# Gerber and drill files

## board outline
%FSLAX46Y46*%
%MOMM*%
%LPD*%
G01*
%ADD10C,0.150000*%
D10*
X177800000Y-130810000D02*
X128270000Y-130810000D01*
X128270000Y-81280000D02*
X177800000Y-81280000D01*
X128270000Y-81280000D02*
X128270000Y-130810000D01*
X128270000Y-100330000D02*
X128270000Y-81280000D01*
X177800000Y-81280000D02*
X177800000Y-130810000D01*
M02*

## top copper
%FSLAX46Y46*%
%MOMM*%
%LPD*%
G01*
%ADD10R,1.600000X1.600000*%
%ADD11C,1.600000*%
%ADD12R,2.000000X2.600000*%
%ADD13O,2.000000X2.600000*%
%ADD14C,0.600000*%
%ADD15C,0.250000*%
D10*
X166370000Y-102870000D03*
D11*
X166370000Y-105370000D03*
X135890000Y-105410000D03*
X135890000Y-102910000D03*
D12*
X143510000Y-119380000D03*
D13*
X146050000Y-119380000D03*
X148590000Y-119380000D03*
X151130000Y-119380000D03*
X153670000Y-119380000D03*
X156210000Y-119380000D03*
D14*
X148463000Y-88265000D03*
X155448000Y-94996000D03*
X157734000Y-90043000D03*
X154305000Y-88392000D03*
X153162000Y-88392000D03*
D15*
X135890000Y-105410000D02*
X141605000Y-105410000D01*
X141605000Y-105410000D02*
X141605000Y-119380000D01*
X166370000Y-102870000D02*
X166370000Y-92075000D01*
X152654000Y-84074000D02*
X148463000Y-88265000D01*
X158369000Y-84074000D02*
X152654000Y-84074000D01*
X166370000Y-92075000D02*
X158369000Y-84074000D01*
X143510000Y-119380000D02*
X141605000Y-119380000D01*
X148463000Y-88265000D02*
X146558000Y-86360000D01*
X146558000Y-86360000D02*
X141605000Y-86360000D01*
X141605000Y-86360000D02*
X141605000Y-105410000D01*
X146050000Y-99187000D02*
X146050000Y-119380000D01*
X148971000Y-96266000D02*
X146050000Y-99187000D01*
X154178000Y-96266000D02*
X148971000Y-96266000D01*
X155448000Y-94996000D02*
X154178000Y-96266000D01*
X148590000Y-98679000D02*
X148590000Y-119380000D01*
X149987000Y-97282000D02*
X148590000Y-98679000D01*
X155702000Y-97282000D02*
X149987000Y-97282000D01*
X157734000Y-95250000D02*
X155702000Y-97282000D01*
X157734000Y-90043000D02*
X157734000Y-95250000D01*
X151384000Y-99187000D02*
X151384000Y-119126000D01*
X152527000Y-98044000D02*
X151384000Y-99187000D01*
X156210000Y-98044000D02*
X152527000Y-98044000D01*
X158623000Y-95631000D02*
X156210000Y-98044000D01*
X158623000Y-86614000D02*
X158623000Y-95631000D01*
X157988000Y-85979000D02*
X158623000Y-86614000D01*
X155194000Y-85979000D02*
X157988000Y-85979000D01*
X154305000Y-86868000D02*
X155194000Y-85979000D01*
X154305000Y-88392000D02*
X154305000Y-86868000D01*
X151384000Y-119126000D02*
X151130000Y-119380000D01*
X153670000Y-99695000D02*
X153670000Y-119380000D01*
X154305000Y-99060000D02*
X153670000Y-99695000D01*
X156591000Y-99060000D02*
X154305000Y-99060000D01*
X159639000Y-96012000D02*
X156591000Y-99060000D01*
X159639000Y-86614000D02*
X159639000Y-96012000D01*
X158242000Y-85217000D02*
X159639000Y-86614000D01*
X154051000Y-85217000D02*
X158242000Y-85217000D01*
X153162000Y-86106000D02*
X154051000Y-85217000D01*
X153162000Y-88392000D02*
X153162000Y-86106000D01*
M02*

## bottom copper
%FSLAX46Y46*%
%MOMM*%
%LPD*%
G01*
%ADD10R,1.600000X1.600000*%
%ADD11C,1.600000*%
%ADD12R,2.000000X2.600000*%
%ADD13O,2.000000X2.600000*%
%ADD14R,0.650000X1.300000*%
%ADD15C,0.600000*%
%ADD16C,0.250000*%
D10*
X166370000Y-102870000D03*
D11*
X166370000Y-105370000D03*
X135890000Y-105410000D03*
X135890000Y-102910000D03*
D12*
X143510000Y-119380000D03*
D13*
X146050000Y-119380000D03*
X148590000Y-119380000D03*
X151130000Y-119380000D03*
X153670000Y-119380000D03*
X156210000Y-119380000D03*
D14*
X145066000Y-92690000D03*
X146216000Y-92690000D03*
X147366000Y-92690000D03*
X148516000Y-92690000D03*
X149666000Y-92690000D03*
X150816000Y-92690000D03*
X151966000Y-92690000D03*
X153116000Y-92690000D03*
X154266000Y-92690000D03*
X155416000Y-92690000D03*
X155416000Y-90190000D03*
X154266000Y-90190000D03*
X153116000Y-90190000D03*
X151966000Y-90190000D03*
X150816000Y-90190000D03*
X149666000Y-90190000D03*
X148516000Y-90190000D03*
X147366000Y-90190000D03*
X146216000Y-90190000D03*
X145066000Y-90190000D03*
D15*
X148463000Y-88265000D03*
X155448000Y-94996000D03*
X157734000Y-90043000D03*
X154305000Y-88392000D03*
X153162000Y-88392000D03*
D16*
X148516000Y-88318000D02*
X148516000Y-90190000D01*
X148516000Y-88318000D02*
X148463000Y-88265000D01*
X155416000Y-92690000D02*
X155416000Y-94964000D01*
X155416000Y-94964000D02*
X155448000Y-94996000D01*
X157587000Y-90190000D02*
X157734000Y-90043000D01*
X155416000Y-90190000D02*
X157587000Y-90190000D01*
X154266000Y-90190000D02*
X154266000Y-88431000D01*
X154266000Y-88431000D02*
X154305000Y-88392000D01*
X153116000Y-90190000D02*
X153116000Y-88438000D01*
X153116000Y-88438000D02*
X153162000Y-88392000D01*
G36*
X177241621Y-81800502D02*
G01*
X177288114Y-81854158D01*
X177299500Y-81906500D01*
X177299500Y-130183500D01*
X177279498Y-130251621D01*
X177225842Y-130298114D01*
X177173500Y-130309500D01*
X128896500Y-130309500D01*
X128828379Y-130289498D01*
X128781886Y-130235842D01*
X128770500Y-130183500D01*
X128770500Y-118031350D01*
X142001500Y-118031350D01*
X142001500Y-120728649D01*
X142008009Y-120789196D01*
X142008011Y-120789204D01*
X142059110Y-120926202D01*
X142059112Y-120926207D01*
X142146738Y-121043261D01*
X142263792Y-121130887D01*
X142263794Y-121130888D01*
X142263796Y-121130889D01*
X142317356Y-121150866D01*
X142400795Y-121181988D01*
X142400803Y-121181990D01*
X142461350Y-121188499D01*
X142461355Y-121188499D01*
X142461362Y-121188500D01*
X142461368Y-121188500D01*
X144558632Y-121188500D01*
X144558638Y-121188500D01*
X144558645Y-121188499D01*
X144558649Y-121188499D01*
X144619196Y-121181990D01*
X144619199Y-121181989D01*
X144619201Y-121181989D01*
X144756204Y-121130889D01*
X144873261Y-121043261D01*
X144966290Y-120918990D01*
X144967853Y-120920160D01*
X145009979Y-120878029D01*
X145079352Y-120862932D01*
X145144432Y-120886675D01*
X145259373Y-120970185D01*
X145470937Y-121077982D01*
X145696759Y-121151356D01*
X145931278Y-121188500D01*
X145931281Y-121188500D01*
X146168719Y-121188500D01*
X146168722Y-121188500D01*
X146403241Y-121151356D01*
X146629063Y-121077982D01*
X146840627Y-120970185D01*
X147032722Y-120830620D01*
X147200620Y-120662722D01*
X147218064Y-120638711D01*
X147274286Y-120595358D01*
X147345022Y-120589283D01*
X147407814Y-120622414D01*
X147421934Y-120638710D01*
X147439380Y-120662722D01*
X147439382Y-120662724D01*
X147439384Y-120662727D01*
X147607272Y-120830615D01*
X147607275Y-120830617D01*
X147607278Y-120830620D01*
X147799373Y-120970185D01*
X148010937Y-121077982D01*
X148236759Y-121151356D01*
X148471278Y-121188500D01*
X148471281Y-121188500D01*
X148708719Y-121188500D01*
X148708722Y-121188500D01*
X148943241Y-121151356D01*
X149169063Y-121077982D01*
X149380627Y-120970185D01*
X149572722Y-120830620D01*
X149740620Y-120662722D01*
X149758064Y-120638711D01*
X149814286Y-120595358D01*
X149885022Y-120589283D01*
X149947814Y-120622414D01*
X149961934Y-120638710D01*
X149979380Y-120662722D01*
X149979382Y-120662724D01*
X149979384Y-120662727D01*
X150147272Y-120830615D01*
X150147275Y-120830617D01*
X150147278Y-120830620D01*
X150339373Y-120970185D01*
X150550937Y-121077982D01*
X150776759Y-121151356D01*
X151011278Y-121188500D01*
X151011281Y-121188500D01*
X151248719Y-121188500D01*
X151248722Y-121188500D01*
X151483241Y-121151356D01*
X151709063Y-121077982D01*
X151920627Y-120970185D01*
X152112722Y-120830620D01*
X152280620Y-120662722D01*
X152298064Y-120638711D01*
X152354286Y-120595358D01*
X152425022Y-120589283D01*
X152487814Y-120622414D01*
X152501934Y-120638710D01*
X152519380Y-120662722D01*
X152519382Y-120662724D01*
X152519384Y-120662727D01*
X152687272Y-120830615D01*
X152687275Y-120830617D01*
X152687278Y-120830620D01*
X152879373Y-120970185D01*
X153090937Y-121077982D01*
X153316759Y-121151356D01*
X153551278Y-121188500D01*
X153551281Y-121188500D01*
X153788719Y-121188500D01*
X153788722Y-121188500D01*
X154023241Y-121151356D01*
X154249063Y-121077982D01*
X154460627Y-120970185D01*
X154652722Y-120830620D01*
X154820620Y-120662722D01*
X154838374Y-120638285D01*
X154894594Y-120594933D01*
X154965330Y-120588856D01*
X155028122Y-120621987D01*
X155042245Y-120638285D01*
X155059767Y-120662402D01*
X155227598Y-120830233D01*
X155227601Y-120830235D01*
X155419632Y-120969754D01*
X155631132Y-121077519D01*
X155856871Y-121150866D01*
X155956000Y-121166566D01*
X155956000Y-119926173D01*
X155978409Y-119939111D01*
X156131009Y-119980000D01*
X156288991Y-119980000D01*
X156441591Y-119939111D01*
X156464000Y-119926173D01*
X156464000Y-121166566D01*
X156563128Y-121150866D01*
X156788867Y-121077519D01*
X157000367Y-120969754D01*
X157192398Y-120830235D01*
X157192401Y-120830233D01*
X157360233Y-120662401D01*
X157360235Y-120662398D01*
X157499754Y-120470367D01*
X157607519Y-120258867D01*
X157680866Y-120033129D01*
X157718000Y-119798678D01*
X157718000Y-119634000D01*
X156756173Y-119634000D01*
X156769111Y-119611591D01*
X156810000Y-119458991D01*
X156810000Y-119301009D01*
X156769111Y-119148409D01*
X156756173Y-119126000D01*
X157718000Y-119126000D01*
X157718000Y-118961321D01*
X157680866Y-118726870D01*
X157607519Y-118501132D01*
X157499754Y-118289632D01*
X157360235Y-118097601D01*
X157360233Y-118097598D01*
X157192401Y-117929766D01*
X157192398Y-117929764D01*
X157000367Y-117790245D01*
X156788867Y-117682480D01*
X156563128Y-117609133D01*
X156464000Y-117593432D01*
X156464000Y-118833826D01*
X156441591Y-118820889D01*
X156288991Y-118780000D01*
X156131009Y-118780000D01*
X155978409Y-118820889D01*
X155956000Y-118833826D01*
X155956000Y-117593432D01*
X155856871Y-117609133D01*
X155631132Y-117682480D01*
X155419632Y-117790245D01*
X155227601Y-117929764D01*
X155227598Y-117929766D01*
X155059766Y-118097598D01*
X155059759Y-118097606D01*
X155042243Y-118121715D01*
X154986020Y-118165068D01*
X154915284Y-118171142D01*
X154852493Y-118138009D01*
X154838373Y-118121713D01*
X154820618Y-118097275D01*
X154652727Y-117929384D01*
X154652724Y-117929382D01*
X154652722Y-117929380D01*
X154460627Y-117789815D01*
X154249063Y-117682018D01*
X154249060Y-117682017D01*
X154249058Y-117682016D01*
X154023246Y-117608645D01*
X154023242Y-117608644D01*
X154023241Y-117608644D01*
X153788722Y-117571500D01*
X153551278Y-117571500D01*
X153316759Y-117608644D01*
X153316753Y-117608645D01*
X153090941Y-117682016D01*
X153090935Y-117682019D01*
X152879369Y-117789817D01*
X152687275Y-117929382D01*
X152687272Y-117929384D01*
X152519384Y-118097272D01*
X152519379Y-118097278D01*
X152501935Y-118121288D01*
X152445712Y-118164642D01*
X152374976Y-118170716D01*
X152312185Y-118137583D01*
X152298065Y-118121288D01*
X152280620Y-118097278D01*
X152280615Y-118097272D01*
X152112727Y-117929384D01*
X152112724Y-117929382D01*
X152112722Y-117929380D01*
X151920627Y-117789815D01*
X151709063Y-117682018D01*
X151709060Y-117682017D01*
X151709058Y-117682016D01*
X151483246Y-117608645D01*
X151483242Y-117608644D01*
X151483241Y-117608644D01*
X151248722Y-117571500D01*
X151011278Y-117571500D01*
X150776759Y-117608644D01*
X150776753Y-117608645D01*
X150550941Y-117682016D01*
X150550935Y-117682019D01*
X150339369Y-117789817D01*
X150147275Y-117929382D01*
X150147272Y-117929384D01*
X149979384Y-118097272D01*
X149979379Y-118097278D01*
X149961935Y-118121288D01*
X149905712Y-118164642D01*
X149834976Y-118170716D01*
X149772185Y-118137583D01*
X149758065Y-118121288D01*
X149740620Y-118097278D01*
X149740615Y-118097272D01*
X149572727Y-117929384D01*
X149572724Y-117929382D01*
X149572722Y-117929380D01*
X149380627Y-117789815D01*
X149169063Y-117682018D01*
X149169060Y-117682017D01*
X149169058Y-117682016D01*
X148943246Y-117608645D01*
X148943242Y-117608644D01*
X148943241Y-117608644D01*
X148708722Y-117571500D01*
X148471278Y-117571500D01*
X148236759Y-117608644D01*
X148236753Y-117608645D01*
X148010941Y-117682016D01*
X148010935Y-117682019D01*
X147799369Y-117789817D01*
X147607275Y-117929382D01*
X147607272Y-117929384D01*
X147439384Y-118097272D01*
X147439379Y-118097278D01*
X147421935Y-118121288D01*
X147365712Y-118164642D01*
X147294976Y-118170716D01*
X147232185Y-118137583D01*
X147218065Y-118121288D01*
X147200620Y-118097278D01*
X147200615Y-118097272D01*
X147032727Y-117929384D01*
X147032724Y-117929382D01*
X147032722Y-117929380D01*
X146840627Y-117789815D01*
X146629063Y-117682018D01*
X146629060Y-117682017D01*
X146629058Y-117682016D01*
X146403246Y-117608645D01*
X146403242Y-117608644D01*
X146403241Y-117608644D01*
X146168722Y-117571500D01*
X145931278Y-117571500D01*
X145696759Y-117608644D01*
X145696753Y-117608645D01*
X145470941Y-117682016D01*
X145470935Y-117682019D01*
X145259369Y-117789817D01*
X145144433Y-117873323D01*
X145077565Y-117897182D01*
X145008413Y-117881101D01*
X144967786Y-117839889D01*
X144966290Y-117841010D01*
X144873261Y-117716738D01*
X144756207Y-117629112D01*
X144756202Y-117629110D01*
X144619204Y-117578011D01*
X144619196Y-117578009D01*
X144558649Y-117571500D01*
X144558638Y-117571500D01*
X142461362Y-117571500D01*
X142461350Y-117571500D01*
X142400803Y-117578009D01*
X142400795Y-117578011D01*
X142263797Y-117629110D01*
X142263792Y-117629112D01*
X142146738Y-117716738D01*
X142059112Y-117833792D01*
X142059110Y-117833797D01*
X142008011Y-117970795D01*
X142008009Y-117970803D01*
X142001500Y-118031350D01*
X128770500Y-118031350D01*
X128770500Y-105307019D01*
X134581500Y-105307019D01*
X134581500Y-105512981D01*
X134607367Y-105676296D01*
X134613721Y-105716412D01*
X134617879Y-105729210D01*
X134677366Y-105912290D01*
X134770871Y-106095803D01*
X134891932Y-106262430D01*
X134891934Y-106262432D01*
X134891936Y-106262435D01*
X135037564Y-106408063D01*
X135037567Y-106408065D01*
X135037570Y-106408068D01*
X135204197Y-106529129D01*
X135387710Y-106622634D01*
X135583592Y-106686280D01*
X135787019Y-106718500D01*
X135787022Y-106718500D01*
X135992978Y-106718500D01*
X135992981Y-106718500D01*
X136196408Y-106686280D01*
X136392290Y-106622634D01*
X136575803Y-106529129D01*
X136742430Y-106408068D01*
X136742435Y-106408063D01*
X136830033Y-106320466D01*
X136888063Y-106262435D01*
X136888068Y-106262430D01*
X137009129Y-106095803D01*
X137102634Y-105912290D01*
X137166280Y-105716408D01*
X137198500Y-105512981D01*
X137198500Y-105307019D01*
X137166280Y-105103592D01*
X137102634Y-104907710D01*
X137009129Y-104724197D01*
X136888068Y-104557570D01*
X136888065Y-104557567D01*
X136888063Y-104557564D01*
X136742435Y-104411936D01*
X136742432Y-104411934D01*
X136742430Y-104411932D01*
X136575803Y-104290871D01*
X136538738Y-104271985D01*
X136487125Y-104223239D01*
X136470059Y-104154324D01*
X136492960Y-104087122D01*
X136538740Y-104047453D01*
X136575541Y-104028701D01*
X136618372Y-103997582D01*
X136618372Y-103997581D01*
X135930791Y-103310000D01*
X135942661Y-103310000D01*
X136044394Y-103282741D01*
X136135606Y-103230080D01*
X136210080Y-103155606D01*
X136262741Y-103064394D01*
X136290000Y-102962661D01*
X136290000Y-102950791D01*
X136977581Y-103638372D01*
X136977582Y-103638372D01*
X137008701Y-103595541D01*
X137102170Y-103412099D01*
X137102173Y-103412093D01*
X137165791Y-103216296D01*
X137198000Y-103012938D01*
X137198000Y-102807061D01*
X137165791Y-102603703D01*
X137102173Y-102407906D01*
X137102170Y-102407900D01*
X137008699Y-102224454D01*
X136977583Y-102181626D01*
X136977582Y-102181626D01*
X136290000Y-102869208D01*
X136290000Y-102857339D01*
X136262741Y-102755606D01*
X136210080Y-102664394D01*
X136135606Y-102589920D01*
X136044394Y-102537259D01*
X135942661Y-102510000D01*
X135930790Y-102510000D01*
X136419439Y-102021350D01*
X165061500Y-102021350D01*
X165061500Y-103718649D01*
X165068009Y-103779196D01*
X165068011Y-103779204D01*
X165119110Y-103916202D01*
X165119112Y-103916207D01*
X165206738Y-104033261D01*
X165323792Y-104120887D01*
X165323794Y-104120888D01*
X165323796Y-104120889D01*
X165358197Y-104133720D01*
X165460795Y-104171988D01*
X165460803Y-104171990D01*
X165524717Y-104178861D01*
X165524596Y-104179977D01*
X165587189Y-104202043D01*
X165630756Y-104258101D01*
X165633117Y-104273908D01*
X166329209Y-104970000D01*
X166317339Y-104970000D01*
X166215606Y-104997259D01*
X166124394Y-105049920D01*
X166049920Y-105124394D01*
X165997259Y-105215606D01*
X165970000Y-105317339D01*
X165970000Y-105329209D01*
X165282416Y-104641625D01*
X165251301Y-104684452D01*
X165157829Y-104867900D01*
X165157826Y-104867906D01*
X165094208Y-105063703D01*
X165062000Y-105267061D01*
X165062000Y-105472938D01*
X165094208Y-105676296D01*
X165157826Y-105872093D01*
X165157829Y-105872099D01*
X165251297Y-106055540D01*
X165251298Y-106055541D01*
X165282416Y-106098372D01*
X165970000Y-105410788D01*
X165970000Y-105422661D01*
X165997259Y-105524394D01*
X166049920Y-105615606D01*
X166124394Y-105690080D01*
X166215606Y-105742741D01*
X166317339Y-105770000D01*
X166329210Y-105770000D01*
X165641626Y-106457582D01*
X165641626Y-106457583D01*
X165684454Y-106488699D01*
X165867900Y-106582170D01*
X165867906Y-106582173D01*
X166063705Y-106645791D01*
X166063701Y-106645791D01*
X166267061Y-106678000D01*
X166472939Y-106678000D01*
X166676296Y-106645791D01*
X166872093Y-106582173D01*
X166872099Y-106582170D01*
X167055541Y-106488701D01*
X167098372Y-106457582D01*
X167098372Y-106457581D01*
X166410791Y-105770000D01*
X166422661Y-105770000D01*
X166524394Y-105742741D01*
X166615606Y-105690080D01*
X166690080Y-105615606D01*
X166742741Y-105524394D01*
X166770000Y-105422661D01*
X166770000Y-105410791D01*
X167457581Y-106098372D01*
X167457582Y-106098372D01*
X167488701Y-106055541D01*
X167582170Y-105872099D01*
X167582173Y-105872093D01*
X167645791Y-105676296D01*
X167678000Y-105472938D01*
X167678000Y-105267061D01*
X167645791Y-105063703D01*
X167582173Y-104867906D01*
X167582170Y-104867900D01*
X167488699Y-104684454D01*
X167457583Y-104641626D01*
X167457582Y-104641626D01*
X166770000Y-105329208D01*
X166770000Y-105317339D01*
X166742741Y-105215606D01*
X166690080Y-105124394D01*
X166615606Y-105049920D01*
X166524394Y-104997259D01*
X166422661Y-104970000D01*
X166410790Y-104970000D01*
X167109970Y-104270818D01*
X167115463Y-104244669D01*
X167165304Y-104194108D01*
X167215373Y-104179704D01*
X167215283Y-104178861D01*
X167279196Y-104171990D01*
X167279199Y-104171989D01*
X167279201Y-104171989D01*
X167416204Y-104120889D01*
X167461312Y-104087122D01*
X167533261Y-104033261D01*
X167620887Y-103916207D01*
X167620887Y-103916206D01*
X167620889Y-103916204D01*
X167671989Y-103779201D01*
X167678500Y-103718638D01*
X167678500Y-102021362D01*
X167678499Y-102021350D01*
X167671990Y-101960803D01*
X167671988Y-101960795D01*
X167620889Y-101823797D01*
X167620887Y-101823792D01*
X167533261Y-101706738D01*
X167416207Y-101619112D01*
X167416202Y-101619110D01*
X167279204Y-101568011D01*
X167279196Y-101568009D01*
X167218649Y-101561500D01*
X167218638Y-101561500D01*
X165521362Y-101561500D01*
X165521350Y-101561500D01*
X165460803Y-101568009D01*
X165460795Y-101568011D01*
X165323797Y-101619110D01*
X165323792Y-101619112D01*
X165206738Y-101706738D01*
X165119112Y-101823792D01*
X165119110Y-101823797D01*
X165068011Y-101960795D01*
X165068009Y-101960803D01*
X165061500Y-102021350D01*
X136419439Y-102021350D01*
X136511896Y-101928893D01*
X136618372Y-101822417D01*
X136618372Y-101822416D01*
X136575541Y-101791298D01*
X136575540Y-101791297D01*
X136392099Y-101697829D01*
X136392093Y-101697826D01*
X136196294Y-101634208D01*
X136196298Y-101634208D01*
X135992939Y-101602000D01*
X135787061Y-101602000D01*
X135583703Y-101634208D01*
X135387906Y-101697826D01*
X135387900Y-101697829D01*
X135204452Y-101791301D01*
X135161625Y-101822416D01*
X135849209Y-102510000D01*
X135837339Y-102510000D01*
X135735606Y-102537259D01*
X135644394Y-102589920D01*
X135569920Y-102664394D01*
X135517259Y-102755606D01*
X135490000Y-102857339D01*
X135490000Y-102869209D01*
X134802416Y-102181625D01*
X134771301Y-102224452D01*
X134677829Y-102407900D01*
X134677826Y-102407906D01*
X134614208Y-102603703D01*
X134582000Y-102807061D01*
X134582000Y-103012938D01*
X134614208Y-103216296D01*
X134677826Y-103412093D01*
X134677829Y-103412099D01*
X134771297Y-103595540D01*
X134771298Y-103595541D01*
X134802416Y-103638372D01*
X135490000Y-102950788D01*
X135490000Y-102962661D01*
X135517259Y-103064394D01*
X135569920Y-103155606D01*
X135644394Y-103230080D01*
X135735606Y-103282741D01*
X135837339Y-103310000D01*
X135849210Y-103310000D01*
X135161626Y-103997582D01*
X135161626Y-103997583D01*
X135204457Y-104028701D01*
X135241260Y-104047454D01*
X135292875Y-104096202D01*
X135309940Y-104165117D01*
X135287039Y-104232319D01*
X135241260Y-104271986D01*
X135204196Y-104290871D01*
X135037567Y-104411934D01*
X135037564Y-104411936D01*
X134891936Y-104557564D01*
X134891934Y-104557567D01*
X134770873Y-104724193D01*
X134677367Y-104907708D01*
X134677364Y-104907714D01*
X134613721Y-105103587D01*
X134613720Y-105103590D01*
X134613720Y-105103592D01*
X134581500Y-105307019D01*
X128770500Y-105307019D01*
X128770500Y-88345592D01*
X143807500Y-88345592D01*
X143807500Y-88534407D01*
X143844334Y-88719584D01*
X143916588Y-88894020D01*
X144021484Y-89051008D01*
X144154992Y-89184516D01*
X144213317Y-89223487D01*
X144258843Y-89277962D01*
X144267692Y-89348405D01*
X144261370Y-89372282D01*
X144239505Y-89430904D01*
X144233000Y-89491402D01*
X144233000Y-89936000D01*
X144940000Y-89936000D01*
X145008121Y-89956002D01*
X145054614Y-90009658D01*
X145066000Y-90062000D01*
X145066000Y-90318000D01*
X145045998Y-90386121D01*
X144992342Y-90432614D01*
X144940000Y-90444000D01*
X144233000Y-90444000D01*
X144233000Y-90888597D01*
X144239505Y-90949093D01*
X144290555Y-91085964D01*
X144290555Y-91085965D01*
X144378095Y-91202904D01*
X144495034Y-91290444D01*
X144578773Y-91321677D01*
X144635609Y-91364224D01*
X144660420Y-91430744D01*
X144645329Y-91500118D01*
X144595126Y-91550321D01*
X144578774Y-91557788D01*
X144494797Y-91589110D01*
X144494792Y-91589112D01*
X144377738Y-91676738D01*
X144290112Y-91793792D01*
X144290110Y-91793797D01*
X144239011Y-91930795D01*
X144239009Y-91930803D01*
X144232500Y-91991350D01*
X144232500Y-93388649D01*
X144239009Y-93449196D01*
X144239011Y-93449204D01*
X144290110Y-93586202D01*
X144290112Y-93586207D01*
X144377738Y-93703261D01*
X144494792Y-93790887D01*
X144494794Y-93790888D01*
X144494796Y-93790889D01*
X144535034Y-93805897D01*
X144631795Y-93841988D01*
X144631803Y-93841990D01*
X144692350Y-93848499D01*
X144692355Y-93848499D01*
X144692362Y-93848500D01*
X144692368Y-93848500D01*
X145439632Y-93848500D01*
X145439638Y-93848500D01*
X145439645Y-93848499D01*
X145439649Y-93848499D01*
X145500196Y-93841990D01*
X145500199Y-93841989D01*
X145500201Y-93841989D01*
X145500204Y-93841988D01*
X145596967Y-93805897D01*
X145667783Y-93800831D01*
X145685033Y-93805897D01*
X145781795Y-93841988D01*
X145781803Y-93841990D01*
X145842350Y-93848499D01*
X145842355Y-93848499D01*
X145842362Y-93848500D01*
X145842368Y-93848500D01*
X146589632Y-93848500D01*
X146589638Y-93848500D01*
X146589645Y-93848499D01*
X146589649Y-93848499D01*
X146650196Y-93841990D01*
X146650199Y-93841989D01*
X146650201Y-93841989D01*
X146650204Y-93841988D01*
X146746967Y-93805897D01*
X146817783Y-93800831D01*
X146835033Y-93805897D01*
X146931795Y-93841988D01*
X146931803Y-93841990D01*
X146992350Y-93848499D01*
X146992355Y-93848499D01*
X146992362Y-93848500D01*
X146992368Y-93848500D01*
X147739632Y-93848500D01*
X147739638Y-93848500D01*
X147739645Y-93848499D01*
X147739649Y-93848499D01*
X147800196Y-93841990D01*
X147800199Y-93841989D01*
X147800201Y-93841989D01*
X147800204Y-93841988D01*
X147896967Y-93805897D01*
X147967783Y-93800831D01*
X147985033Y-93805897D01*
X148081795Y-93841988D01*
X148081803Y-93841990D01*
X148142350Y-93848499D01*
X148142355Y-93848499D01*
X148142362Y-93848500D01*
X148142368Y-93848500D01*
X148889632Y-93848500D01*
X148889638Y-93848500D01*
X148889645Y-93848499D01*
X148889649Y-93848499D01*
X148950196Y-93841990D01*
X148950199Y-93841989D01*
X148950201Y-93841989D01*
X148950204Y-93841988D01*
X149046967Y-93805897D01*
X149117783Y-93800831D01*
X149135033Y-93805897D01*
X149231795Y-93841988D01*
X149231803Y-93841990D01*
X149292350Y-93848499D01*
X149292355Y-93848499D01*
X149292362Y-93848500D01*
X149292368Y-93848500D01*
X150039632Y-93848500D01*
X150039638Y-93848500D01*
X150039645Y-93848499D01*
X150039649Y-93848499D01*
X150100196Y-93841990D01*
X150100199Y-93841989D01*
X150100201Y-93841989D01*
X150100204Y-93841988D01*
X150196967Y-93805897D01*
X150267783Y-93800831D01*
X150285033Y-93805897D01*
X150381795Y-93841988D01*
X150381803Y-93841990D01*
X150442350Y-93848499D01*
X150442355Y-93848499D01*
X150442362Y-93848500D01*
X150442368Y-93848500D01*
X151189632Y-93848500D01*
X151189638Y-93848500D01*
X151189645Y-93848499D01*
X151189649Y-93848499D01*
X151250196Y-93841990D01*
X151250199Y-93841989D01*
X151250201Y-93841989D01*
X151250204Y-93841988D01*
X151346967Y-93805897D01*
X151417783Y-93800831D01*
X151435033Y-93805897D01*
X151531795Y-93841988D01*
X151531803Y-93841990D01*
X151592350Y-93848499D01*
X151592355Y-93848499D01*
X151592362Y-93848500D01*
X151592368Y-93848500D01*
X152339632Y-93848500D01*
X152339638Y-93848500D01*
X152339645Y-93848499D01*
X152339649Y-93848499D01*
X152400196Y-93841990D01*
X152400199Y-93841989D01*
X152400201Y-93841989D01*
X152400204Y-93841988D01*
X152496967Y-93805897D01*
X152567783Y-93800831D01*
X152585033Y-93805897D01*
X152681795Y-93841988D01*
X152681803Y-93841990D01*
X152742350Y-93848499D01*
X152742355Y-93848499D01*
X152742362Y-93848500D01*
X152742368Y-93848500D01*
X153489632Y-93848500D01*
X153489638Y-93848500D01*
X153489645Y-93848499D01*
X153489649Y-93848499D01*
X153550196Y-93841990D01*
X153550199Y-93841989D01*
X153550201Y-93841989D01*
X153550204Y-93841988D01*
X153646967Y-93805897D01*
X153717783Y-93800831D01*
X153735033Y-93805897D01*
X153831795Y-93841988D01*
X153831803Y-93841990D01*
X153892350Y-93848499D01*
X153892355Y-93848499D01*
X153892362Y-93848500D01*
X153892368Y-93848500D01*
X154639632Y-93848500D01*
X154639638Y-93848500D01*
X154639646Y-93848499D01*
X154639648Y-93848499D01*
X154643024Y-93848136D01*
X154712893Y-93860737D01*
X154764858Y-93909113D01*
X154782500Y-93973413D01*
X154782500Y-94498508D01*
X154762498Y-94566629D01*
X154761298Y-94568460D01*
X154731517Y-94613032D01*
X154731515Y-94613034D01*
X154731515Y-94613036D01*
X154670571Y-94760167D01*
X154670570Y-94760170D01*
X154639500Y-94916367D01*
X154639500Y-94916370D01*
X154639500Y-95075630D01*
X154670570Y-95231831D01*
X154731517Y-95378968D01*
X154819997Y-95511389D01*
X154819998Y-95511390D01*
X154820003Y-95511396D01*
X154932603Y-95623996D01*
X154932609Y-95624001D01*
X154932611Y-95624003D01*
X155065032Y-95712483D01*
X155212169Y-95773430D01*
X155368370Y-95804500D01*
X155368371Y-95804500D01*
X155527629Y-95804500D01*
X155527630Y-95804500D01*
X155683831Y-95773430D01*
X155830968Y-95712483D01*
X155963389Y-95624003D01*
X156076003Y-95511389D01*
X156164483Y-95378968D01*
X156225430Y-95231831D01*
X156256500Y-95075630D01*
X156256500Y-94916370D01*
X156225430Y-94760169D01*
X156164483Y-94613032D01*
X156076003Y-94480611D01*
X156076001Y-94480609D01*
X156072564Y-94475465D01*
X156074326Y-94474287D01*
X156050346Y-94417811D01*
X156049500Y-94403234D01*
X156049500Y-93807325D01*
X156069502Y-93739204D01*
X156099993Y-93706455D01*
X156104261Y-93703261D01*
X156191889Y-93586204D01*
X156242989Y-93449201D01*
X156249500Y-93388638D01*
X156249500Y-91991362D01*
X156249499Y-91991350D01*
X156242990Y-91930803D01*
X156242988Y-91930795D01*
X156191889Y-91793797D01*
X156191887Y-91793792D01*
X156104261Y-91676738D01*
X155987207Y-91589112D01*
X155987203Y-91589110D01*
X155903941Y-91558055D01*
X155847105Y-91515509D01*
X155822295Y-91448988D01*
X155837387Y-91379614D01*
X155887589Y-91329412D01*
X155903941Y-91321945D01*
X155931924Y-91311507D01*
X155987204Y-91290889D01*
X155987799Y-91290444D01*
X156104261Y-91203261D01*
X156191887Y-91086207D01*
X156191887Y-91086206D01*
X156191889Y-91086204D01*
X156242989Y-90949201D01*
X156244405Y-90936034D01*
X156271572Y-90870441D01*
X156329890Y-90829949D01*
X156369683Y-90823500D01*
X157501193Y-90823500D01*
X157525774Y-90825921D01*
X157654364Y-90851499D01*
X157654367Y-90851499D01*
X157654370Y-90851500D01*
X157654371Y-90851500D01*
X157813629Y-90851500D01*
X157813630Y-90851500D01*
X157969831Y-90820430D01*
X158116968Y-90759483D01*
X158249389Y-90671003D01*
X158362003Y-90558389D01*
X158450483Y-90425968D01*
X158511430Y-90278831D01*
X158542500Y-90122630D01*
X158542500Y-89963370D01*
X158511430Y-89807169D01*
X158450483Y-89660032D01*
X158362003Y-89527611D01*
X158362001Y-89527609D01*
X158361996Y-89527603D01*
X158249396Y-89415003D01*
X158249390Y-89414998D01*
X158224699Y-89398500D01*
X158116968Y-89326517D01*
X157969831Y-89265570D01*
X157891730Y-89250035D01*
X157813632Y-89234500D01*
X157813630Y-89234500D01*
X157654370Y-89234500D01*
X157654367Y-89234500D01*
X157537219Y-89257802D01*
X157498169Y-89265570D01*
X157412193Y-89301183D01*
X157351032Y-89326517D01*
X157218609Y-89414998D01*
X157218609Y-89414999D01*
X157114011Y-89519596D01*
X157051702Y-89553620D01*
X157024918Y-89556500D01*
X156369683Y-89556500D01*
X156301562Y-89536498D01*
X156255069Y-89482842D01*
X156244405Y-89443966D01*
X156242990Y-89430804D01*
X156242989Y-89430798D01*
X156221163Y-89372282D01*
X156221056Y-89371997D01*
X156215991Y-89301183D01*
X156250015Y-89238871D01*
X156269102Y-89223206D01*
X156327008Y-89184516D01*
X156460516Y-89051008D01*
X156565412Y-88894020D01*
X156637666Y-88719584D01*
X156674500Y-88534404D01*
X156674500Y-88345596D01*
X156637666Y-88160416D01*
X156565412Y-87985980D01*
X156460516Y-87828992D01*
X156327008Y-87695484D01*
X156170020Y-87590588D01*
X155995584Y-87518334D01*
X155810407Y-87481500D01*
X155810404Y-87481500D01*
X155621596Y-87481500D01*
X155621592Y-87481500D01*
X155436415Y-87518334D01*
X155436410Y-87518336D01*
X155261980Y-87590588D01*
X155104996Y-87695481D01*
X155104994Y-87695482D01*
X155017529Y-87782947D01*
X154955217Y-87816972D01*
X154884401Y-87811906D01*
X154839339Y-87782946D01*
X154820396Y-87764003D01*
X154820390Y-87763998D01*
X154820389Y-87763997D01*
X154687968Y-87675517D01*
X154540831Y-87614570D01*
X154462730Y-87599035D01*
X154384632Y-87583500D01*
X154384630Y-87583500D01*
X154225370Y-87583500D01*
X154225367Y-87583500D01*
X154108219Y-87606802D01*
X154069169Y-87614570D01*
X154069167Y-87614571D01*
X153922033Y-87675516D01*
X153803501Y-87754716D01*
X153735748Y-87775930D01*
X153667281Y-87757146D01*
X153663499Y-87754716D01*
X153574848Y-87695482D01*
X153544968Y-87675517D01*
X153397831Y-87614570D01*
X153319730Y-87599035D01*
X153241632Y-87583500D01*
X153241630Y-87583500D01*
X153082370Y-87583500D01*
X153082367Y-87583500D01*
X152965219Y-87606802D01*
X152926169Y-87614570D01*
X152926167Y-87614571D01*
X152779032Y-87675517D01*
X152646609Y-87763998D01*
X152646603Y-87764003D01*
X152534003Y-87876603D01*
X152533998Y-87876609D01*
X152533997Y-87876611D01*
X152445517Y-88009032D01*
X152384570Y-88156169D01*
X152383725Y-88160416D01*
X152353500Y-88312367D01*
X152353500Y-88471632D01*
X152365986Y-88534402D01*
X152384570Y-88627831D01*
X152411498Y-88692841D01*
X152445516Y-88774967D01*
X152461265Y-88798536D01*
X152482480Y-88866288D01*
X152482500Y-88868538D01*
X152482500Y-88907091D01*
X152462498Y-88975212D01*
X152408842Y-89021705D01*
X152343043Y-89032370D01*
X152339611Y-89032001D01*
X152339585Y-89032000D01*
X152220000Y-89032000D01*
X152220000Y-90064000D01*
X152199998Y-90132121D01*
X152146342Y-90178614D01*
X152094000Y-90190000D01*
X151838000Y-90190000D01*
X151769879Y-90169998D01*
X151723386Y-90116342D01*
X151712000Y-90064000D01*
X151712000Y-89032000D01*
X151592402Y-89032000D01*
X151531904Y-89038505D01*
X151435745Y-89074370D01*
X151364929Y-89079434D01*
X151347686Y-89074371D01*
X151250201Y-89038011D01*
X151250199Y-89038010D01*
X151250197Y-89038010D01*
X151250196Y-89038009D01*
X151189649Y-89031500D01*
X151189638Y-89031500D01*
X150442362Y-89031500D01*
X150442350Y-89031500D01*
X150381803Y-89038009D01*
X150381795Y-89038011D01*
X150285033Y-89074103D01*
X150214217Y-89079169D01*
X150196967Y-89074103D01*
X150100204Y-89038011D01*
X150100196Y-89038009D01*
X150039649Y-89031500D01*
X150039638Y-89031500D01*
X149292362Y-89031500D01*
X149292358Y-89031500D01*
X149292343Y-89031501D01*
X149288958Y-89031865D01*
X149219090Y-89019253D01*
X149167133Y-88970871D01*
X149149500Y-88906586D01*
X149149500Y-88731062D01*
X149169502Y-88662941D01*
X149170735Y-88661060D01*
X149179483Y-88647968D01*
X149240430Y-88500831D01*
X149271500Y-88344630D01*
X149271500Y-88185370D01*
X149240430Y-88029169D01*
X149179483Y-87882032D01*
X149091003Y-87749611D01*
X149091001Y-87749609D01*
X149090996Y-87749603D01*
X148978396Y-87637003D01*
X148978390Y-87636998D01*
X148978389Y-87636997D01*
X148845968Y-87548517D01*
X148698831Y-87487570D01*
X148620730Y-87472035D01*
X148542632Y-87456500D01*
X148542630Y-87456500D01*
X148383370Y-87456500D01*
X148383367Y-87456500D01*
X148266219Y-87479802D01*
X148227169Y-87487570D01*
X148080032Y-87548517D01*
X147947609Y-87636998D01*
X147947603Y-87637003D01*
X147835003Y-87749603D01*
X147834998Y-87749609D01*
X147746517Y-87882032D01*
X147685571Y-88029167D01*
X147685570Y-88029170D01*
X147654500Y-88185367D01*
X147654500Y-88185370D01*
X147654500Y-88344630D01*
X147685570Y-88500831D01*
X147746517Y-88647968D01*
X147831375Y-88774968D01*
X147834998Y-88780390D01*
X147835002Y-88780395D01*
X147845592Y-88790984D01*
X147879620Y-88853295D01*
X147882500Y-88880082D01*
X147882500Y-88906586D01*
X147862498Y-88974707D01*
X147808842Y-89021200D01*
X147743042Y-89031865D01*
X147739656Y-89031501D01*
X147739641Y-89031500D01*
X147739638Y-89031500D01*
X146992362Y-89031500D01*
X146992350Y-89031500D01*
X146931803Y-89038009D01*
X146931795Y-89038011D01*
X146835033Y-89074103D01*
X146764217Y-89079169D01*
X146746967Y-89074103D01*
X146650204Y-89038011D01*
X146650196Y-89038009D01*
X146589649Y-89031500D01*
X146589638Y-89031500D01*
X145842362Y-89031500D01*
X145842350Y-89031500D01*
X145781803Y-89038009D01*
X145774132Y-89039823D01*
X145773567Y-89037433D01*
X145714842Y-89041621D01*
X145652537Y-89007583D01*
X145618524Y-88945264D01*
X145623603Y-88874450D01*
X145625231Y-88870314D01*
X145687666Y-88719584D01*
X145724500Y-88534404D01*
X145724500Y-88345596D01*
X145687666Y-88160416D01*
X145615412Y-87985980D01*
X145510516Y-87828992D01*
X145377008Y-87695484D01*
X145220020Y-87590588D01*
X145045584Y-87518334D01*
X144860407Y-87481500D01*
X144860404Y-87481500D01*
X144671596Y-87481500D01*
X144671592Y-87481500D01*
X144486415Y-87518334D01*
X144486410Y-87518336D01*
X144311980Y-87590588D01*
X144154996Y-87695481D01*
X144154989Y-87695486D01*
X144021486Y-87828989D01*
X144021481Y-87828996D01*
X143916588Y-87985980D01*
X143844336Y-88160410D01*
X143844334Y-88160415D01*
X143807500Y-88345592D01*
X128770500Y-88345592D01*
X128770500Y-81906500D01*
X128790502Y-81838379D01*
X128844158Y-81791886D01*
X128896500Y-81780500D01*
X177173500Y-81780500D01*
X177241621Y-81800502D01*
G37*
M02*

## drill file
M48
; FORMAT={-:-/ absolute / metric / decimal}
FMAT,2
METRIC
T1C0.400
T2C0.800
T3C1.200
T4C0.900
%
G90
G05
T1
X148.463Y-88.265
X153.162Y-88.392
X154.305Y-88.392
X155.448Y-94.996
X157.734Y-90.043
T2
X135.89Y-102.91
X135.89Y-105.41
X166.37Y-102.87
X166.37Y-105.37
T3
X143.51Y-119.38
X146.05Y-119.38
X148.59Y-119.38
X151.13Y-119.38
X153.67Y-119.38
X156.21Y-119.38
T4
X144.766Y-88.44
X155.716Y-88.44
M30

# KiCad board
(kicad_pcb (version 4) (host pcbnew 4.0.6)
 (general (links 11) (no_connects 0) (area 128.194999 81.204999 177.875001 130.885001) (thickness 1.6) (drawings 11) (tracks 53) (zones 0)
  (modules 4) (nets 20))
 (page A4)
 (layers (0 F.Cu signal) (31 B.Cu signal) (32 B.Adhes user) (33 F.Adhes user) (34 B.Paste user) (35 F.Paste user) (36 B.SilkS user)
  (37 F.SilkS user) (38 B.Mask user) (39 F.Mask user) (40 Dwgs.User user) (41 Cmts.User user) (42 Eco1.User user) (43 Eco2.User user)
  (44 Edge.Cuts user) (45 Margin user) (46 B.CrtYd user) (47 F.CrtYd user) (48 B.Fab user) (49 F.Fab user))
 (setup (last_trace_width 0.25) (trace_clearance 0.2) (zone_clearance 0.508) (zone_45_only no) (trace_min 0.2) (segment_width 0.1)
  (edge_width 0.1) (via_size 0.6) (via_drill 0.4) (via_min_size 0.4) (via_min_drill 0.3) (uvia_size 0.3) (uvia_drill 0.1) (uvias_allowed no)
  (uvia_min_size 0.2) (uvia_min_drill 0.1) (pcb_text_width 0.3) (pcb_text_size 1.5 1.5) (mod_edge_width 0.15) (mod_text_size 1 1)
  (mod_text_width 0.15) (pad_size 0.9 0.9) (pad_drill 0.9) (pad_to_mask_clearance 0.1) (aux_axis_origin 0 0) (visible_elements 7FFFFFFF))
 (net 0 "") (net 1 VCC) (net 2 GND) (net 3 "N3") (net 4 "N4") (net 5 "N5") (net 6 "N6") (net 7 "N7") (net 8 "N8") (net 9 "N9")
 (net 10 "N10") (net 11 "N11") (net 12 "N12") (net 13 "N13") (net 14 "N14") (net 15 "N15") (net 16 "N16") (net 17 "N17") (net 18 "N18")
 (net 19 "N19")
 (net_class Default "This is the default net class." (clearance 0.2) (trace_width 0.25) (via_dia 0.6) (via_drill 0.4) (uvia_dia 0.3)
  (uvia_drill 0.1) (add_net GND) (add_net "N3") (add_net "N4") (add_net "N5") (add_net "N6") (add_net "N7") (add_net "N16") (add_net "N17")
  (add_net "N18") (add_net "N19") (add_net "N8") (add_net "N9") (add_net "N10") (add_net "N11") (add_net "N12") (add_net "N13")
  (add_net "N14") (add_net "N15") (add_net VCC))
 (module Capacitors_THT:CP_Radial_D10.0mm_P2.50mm (layer F.Cu) (at 166.37 102.87 270)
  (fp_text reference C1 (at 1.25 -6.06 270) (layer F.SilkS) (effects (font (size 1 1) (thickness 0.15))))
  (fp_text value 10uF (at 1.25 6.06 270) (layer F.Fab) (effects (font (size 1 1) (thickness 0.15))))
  (pad 1 thru_hole rect (at 0 0 270) (size 1.6 1.6) (drill 0.8) (layers *.Cu *.Mask) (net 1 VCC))
  (pad 2 thru_hole circle (at 2.5 0 270) (size 1.6 1.6) (drill 0.8) (layers *.Cu *.Mask) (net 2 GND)))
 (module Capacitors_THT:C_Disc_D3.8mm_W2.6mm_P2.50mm (layer F.Cu) (at 135.89 105.41 90)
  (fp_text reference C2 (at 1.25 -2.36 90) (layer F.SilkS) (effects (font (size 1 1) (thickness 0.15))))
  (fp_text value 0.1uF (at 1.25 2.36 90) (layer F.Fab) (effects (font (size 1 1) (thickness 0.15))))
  (pad 1 thru_hole circle (at 0 0 90) (size 1.6 1.6) (drill 0.8) (layers *.Cu *.Mask) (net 1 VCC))
  (pad 2 thru_hole circle (at 2.5 0 90) (size 1.6 1.6) (drill 0.8) (layers *.Cu *.Mask) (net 2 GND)))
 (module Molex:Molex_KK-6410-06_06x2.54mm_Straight (layer F.Cu) (at 143.51 119.38)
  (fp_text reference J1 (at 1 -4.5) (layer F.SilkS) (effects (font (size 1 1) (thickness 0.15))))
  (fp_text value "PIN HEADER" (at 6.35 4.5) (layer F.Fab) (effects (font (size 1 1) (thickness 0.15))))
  (pad 1 thru_hole rect (at 0 0) (size 2 2.6) (drill 1.2) (layers *.Cu *.Mask) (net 1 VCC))
  (pad 2 thru_hole oval (at 2.54 0) (size 2 2.6) (drill 1.2) (layers *.Cu *.Mask) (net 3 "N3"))
  (pad 3 thru_hole oval (at 5.08 0) (size 2 2.6) (drill 1.2) (layers *.Cu *.Mask) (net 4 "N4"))
  (pad 4 thru_hole oval (at 7.62 0) (size 2 2.6) (drill 1.2) (layers *.Cu *.Mask) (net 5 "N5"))
  (pad 5 thru_hole oval (at 10.16 0) (size 2 2.6) (drill 1.2) (layers *.Cu *.Mask) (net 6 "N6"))
  (pad 6 thru_hole oval (at 12.7 0) (size 2 2.6) (drill 1.2) (layers *.Cu *.Mask) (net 2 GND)))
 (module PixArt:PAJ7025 (layer F.Cu) (at 150.241 91.44)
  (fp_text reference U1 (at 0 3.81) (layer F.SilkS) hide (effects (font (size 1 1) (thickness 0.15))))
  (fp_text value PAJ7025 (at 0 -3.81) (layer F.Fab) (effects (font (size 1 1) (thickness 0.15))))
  (pad "" np_thru_hole oval (at -5.475 -3) (size 0.9 0.9) (drill 0.9) (layers *.Cu))
  (pad 1 smd rect (at -5.175 1.25) (size 0.65 1.3) (layers B.Cu B.Paste B.Mask) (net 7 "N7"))
  (pad 2 smd rect (at -4.025 1.25) (size 0.65 1.3) (layers B.Cu B.Paste B.Mask) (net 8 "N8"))
  (pad 3 smd rect (at -2.875 1.25) (size 0.65 1.3) (layers B.Cu B.Paste B.Mask) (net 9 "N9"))
  (pad 4 smd rect (at -1.725 1.25) (size 0.65 1.3) (layers B.Cu B.Paste B.Mask) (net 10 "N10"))
  (pad 5 smd rect (at -0.575 1.25) (size 0.65 1.3) (layers B.Cu B.Paste B.Mask) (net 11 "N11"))
  (pad 6 smd rect (at 0.575 1.25) (size 0.65 1.3) (layers B.Cu B.Paste B.Mask) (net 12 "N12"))
  (pad 7 smd rect (at 1.725 1.25) (size 0.65 1.3) (layers B.Cu B.Paste B.Mask) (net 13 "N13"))
  (pad 8 smd rect (at 2.875 1.25) (size 0.65 1.3) (layers B.Cu B.Paste B.Mask) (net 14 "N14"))
  (pad 9 smd rect (at 4.025 1.25) (size 0.65 1.3) (layers B.Cu B.Paste B.Mask) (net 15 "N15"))
  (pad 10 smd rect (at 5.175 1.25) (size 0.65 1.3) (layers B.Cu B.Paste B.Mask) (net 3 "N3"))
  (pad 11 smd rect (at 5.175 -1.25) (size 0.65 1.3) (layers B.Cu B.Paste B.Mask) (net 4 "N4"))
  (pad 12 smd rect (at 4.025 -1.25) (size 0.65 1.3) (layers B.Cu B.Paste B.Mask) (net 5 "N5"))
  (pad 13 smd rect (at 2.875 -1.25) (size 0.65 1.3) (layers B.Cu B.Paste B.Mask) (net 6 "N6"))
  (pad 14 smd rect (at 1.725 -1.25) (size 0.65 1.3) (layers B.Cu B.Paste B.Mask) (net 2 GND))
  (pad 15 smd rect (at 0.575 -1.25) (size 0.65 1.3) (layers B.Cu B.Paste B.Mask) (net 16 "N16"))
  (pad 16 smd rect (at -0.575 -1.25) (size 0.65 1.3) (layers B.Cu B.Paste B.Mask) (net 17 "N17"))
  (pad 17 smd rect (at -1.725 -1.25) (size 0.65 1.3) (layers B.Cu B.Paste B.Mask) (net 1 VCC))
  (pad 18 smd rect (at -2.875 -1.25) (size 0.65 1.3) (layers B.Cu B.Paste B.Mask) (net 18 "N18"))
  (pad 19 smd rect (at -4.025 -1.25) (size 0.65 1.3) (layers B.Cu B.Paste B.Mask) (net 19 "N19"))
  (pad 20 smd rect (at -5.175 -1.25) (size 0.65 1.3) (layers B.Cu B.Paste B.Mask) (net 2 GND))
  (pad "" np_thru_hole oval (at 5.475 -3) (size 0.9 0.9) (drill 0.9) (layers *.Cu)))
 (gr_line (start 177.8 130.81) (end 128.27 130.81) (angle 90) (layer Edge.Cuts) (width 0.15))
 (gr_line (start 128.27 81.28) (end 177.8 81.28) (angle 90) (layer Edge.Cuts) (width 0.15))
 (gr_line (start 128.27 81.28) (end 128.27 130.81) (angle 90) (layer Edge.Cuts) (width 0.15))
 (gr_line (start 128.27 100.33) (end 128.27 81.28) (angle 90) (layer Edge.Cuts) (width 0.15))
 (gr_line (start 177.8 81.28) (end 177.8 130.81) (angle 90) (layer Edge.Cuts) (width 0.15))
 (segment (start 135.89 105.41) (end 141.605 105.41) (width 0.25) (layer F.Cu) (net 1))
 (segment (start 141.605 105.41) (end 141.605 119.38) (width 0.25) (layer F.Cu) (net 1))
 (segment (start 166.37 102.87) (end 166.37 92.075) (width 0.25) (layer F.Cu) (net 1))
 (segment (start 152.654 84.074) (end 148.463 88.265) (width 0.25) (layer F.Cu) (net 1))
 (segment (start 158.369 84.074) (end 152.654 84.074) (width 0.25) (layer F.Cu) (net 1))
 (segment (start 166.37 92.075) (end 158.369 84.074) (width 0.25) (layer F.Cu) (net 1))
 (segment (start 143.51 119.38) (end 141.605 119.38) (width 0.25) (layer F.Cu) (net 1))
 (segment (start 148.516 88.318) (end 148.516 90.19) (width 0.25) (layer B.Cu) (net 1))
 (segment (start 148.516 88.318) (end 148.463 88.265) (width 0.25) (layer B.Cu) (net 1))
 (via (at 148.463 88.265) (size 0.6) (drill 0.4) (layers F.Cu B.Cu) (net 1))
 (segment (start 148.463 88.265) (end 146.558 86.36) (width 0.25) (layer F.Cu) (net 1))
 (segment (start 146.558 86.36) (end 141.605 86.36) (width 0.25) (layer F.Cu) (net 1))
 (segment (start 141.605 86.36) (end 141.605 105.41) (width 0.25) (layer F.Cu) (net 1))
 (segment (start 155.416 92.69) (end 155.416 94.964) (width 0.25) (layer B.Cu) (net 3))
 (segment (start 146.05 99.187) (end 146.05 119.38) (width 0.25) (layer F.Cu) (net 3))
 (segment (start 148.971 96.266) (end 146.05 99.187) (width 0.25) (layer F.Cu) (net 3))
 (segment (start 154.178 96.266) (end 148.971 96.266) (width 0.25) (layer F.Cu) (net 3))
 (segment (start 155.448 94.996) (end 154.178 96.266) (width 0.25) (layer F.Cu) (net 3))
 (via (at 155.448 94.996) (size 0.6) (drill 0.4) (layers F.Cu B.Cu) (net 3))
 (segment (start 155.416 94.964) (end 155.448 94.996) (width 0.25) (layer B.Cu) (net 3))
 (segment (start 148.59 98.679) (end 148.59 119.38) (width 0.25) (layer F.Cu) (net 4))
 (segment (start 149.987 97.282) (end 148.59 98.679) (width 0.25) (layer F.Cu) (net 4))
 (segment (start 155.702 97.282) (end 149.987 97.282) (width 0.25) (layer F.Cu) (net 4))
 (segment (start 157.734 95.25) (end 155.702 97.282) (width 0.25) (layer F.Cu) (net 4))
 (segment (start 157.734 90.043) (end 157.734 95.25) (width 0.25) (layer F.Cu) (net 4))
 (via (at 157.734 90.043) (size 0.6) (drill 0.4) (layers F.Cu B.Cu) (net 4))
 (segment (start 157.587 90.19) (end 157.734 90.043) (width 0.25) (layer B.Cu) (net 4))
 (segment (start 155.416 90.19) (end 157.587 90.19) (width 0.25) (layer B.Cu) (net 4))
 (segment (start 154.266 90.19) (end 154.266 88.431) (width 0.25) (layer B.Cu) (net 5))
 (segment (start 151.384 99.187) (end 151.384 119.126) (width 0.25) (layer F.Cu) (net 5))
 (segment (start 152.527 98.044) (end 151.384 99.187) (width 0.25) (layer F.Cu) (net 5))
 (segment (start 156.21 98.044) (end 152.527 98.044) (width 0.25) (layer F.Cu) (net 5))
 (segment (start 158.623 95.631) (end 156.21 98.044) (width 0.25) (layer F.Cu) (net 5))
 (segment (start 158.623 86.614) (end 158.623 95.631) (width 0.25) (layer F.Cu) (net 5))
 (segment (start 157.988 85.979) (end 158.623 86.614) (width 0.25) (layer F.Cu) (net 5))
 (segment (start 155.194 85.979) (end 157.988 85.979) (width 0.25) (layer F.Cu) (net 5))
 (segment (start 154.305 86.868) (end 155.194 85.979) (width 0.25) (layer F.Cu) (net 5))
 (segment (start 154.305 88.392) (end 154.305 86.868) (width 0.25) (layer F.Cu) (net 5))
 (via (at 154.305 88.392) (size 0.6) (drill 0.4) (layers F.Cu B.Cu) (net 5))
 (segment (start 154.266 88.431) (end 154.305 88.392) (width 0.25) (layer B.Cu) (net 5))
 (segment (start 151.384 119.126) (end 151.13 119.38) (width 0.25) (layer F.Cu) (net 5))
 (segment (start 153.116 90.19) (end 153.116 88.438) (width 0.25) (layer B.Cu) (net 6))
 (segment (start 153.67 99.695) (end 153.67 119.38) (width 0.25) (layer F.Cu) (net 6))
 (segment (start 154.305 99.06) (end 153.67 99.695) (width 0.25) (layer F.Cu) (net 6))
 (segment (start 156.591 99.06) (end 154.305 99.06) (width 0.25) (layer F.Cu) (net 6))
 (segment (start 159.639 96.012) (end 156.591 99.06) (width 0.25) (layer F.Cu) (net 6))
 (segment (start 159.639 86.614) (end 159.639 96.012) (width 0.25) (layer F.Cu) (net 6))
 (segment (start 158.242 85.217) (end 159.639 86.614) (width 0.25) (layer F.Cu) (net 6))
 (segment (start 154.051 85.217) (end 158.242 85.217) (width 0.25) (layer F.Cu) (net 6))
 (segment (start 153.162 86.106) (end 154.051 85.217) (width 0.25) (layer F.Cu) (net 6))
 (segment (start 153.162 88.392) (end 153.162 86.106) (width 0.25) (layer F.Cu) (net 6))
 (via (at 153.162 88.392) (size 0.6) (drill 0.4) (layers F.Cu B.Cu) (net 6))
 (segment (start 153.116 88.438) (end 153.162 88.392) (width 0.25) (layer B.Cu) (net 6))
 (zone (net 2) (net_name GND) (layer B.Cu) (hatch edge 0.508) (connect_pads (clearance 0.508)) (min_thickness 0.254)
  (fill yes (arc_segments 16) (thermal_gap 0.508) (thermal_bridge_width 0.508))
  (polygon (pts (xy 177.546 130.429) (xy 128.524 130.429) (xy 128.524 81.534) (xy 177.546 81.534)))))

